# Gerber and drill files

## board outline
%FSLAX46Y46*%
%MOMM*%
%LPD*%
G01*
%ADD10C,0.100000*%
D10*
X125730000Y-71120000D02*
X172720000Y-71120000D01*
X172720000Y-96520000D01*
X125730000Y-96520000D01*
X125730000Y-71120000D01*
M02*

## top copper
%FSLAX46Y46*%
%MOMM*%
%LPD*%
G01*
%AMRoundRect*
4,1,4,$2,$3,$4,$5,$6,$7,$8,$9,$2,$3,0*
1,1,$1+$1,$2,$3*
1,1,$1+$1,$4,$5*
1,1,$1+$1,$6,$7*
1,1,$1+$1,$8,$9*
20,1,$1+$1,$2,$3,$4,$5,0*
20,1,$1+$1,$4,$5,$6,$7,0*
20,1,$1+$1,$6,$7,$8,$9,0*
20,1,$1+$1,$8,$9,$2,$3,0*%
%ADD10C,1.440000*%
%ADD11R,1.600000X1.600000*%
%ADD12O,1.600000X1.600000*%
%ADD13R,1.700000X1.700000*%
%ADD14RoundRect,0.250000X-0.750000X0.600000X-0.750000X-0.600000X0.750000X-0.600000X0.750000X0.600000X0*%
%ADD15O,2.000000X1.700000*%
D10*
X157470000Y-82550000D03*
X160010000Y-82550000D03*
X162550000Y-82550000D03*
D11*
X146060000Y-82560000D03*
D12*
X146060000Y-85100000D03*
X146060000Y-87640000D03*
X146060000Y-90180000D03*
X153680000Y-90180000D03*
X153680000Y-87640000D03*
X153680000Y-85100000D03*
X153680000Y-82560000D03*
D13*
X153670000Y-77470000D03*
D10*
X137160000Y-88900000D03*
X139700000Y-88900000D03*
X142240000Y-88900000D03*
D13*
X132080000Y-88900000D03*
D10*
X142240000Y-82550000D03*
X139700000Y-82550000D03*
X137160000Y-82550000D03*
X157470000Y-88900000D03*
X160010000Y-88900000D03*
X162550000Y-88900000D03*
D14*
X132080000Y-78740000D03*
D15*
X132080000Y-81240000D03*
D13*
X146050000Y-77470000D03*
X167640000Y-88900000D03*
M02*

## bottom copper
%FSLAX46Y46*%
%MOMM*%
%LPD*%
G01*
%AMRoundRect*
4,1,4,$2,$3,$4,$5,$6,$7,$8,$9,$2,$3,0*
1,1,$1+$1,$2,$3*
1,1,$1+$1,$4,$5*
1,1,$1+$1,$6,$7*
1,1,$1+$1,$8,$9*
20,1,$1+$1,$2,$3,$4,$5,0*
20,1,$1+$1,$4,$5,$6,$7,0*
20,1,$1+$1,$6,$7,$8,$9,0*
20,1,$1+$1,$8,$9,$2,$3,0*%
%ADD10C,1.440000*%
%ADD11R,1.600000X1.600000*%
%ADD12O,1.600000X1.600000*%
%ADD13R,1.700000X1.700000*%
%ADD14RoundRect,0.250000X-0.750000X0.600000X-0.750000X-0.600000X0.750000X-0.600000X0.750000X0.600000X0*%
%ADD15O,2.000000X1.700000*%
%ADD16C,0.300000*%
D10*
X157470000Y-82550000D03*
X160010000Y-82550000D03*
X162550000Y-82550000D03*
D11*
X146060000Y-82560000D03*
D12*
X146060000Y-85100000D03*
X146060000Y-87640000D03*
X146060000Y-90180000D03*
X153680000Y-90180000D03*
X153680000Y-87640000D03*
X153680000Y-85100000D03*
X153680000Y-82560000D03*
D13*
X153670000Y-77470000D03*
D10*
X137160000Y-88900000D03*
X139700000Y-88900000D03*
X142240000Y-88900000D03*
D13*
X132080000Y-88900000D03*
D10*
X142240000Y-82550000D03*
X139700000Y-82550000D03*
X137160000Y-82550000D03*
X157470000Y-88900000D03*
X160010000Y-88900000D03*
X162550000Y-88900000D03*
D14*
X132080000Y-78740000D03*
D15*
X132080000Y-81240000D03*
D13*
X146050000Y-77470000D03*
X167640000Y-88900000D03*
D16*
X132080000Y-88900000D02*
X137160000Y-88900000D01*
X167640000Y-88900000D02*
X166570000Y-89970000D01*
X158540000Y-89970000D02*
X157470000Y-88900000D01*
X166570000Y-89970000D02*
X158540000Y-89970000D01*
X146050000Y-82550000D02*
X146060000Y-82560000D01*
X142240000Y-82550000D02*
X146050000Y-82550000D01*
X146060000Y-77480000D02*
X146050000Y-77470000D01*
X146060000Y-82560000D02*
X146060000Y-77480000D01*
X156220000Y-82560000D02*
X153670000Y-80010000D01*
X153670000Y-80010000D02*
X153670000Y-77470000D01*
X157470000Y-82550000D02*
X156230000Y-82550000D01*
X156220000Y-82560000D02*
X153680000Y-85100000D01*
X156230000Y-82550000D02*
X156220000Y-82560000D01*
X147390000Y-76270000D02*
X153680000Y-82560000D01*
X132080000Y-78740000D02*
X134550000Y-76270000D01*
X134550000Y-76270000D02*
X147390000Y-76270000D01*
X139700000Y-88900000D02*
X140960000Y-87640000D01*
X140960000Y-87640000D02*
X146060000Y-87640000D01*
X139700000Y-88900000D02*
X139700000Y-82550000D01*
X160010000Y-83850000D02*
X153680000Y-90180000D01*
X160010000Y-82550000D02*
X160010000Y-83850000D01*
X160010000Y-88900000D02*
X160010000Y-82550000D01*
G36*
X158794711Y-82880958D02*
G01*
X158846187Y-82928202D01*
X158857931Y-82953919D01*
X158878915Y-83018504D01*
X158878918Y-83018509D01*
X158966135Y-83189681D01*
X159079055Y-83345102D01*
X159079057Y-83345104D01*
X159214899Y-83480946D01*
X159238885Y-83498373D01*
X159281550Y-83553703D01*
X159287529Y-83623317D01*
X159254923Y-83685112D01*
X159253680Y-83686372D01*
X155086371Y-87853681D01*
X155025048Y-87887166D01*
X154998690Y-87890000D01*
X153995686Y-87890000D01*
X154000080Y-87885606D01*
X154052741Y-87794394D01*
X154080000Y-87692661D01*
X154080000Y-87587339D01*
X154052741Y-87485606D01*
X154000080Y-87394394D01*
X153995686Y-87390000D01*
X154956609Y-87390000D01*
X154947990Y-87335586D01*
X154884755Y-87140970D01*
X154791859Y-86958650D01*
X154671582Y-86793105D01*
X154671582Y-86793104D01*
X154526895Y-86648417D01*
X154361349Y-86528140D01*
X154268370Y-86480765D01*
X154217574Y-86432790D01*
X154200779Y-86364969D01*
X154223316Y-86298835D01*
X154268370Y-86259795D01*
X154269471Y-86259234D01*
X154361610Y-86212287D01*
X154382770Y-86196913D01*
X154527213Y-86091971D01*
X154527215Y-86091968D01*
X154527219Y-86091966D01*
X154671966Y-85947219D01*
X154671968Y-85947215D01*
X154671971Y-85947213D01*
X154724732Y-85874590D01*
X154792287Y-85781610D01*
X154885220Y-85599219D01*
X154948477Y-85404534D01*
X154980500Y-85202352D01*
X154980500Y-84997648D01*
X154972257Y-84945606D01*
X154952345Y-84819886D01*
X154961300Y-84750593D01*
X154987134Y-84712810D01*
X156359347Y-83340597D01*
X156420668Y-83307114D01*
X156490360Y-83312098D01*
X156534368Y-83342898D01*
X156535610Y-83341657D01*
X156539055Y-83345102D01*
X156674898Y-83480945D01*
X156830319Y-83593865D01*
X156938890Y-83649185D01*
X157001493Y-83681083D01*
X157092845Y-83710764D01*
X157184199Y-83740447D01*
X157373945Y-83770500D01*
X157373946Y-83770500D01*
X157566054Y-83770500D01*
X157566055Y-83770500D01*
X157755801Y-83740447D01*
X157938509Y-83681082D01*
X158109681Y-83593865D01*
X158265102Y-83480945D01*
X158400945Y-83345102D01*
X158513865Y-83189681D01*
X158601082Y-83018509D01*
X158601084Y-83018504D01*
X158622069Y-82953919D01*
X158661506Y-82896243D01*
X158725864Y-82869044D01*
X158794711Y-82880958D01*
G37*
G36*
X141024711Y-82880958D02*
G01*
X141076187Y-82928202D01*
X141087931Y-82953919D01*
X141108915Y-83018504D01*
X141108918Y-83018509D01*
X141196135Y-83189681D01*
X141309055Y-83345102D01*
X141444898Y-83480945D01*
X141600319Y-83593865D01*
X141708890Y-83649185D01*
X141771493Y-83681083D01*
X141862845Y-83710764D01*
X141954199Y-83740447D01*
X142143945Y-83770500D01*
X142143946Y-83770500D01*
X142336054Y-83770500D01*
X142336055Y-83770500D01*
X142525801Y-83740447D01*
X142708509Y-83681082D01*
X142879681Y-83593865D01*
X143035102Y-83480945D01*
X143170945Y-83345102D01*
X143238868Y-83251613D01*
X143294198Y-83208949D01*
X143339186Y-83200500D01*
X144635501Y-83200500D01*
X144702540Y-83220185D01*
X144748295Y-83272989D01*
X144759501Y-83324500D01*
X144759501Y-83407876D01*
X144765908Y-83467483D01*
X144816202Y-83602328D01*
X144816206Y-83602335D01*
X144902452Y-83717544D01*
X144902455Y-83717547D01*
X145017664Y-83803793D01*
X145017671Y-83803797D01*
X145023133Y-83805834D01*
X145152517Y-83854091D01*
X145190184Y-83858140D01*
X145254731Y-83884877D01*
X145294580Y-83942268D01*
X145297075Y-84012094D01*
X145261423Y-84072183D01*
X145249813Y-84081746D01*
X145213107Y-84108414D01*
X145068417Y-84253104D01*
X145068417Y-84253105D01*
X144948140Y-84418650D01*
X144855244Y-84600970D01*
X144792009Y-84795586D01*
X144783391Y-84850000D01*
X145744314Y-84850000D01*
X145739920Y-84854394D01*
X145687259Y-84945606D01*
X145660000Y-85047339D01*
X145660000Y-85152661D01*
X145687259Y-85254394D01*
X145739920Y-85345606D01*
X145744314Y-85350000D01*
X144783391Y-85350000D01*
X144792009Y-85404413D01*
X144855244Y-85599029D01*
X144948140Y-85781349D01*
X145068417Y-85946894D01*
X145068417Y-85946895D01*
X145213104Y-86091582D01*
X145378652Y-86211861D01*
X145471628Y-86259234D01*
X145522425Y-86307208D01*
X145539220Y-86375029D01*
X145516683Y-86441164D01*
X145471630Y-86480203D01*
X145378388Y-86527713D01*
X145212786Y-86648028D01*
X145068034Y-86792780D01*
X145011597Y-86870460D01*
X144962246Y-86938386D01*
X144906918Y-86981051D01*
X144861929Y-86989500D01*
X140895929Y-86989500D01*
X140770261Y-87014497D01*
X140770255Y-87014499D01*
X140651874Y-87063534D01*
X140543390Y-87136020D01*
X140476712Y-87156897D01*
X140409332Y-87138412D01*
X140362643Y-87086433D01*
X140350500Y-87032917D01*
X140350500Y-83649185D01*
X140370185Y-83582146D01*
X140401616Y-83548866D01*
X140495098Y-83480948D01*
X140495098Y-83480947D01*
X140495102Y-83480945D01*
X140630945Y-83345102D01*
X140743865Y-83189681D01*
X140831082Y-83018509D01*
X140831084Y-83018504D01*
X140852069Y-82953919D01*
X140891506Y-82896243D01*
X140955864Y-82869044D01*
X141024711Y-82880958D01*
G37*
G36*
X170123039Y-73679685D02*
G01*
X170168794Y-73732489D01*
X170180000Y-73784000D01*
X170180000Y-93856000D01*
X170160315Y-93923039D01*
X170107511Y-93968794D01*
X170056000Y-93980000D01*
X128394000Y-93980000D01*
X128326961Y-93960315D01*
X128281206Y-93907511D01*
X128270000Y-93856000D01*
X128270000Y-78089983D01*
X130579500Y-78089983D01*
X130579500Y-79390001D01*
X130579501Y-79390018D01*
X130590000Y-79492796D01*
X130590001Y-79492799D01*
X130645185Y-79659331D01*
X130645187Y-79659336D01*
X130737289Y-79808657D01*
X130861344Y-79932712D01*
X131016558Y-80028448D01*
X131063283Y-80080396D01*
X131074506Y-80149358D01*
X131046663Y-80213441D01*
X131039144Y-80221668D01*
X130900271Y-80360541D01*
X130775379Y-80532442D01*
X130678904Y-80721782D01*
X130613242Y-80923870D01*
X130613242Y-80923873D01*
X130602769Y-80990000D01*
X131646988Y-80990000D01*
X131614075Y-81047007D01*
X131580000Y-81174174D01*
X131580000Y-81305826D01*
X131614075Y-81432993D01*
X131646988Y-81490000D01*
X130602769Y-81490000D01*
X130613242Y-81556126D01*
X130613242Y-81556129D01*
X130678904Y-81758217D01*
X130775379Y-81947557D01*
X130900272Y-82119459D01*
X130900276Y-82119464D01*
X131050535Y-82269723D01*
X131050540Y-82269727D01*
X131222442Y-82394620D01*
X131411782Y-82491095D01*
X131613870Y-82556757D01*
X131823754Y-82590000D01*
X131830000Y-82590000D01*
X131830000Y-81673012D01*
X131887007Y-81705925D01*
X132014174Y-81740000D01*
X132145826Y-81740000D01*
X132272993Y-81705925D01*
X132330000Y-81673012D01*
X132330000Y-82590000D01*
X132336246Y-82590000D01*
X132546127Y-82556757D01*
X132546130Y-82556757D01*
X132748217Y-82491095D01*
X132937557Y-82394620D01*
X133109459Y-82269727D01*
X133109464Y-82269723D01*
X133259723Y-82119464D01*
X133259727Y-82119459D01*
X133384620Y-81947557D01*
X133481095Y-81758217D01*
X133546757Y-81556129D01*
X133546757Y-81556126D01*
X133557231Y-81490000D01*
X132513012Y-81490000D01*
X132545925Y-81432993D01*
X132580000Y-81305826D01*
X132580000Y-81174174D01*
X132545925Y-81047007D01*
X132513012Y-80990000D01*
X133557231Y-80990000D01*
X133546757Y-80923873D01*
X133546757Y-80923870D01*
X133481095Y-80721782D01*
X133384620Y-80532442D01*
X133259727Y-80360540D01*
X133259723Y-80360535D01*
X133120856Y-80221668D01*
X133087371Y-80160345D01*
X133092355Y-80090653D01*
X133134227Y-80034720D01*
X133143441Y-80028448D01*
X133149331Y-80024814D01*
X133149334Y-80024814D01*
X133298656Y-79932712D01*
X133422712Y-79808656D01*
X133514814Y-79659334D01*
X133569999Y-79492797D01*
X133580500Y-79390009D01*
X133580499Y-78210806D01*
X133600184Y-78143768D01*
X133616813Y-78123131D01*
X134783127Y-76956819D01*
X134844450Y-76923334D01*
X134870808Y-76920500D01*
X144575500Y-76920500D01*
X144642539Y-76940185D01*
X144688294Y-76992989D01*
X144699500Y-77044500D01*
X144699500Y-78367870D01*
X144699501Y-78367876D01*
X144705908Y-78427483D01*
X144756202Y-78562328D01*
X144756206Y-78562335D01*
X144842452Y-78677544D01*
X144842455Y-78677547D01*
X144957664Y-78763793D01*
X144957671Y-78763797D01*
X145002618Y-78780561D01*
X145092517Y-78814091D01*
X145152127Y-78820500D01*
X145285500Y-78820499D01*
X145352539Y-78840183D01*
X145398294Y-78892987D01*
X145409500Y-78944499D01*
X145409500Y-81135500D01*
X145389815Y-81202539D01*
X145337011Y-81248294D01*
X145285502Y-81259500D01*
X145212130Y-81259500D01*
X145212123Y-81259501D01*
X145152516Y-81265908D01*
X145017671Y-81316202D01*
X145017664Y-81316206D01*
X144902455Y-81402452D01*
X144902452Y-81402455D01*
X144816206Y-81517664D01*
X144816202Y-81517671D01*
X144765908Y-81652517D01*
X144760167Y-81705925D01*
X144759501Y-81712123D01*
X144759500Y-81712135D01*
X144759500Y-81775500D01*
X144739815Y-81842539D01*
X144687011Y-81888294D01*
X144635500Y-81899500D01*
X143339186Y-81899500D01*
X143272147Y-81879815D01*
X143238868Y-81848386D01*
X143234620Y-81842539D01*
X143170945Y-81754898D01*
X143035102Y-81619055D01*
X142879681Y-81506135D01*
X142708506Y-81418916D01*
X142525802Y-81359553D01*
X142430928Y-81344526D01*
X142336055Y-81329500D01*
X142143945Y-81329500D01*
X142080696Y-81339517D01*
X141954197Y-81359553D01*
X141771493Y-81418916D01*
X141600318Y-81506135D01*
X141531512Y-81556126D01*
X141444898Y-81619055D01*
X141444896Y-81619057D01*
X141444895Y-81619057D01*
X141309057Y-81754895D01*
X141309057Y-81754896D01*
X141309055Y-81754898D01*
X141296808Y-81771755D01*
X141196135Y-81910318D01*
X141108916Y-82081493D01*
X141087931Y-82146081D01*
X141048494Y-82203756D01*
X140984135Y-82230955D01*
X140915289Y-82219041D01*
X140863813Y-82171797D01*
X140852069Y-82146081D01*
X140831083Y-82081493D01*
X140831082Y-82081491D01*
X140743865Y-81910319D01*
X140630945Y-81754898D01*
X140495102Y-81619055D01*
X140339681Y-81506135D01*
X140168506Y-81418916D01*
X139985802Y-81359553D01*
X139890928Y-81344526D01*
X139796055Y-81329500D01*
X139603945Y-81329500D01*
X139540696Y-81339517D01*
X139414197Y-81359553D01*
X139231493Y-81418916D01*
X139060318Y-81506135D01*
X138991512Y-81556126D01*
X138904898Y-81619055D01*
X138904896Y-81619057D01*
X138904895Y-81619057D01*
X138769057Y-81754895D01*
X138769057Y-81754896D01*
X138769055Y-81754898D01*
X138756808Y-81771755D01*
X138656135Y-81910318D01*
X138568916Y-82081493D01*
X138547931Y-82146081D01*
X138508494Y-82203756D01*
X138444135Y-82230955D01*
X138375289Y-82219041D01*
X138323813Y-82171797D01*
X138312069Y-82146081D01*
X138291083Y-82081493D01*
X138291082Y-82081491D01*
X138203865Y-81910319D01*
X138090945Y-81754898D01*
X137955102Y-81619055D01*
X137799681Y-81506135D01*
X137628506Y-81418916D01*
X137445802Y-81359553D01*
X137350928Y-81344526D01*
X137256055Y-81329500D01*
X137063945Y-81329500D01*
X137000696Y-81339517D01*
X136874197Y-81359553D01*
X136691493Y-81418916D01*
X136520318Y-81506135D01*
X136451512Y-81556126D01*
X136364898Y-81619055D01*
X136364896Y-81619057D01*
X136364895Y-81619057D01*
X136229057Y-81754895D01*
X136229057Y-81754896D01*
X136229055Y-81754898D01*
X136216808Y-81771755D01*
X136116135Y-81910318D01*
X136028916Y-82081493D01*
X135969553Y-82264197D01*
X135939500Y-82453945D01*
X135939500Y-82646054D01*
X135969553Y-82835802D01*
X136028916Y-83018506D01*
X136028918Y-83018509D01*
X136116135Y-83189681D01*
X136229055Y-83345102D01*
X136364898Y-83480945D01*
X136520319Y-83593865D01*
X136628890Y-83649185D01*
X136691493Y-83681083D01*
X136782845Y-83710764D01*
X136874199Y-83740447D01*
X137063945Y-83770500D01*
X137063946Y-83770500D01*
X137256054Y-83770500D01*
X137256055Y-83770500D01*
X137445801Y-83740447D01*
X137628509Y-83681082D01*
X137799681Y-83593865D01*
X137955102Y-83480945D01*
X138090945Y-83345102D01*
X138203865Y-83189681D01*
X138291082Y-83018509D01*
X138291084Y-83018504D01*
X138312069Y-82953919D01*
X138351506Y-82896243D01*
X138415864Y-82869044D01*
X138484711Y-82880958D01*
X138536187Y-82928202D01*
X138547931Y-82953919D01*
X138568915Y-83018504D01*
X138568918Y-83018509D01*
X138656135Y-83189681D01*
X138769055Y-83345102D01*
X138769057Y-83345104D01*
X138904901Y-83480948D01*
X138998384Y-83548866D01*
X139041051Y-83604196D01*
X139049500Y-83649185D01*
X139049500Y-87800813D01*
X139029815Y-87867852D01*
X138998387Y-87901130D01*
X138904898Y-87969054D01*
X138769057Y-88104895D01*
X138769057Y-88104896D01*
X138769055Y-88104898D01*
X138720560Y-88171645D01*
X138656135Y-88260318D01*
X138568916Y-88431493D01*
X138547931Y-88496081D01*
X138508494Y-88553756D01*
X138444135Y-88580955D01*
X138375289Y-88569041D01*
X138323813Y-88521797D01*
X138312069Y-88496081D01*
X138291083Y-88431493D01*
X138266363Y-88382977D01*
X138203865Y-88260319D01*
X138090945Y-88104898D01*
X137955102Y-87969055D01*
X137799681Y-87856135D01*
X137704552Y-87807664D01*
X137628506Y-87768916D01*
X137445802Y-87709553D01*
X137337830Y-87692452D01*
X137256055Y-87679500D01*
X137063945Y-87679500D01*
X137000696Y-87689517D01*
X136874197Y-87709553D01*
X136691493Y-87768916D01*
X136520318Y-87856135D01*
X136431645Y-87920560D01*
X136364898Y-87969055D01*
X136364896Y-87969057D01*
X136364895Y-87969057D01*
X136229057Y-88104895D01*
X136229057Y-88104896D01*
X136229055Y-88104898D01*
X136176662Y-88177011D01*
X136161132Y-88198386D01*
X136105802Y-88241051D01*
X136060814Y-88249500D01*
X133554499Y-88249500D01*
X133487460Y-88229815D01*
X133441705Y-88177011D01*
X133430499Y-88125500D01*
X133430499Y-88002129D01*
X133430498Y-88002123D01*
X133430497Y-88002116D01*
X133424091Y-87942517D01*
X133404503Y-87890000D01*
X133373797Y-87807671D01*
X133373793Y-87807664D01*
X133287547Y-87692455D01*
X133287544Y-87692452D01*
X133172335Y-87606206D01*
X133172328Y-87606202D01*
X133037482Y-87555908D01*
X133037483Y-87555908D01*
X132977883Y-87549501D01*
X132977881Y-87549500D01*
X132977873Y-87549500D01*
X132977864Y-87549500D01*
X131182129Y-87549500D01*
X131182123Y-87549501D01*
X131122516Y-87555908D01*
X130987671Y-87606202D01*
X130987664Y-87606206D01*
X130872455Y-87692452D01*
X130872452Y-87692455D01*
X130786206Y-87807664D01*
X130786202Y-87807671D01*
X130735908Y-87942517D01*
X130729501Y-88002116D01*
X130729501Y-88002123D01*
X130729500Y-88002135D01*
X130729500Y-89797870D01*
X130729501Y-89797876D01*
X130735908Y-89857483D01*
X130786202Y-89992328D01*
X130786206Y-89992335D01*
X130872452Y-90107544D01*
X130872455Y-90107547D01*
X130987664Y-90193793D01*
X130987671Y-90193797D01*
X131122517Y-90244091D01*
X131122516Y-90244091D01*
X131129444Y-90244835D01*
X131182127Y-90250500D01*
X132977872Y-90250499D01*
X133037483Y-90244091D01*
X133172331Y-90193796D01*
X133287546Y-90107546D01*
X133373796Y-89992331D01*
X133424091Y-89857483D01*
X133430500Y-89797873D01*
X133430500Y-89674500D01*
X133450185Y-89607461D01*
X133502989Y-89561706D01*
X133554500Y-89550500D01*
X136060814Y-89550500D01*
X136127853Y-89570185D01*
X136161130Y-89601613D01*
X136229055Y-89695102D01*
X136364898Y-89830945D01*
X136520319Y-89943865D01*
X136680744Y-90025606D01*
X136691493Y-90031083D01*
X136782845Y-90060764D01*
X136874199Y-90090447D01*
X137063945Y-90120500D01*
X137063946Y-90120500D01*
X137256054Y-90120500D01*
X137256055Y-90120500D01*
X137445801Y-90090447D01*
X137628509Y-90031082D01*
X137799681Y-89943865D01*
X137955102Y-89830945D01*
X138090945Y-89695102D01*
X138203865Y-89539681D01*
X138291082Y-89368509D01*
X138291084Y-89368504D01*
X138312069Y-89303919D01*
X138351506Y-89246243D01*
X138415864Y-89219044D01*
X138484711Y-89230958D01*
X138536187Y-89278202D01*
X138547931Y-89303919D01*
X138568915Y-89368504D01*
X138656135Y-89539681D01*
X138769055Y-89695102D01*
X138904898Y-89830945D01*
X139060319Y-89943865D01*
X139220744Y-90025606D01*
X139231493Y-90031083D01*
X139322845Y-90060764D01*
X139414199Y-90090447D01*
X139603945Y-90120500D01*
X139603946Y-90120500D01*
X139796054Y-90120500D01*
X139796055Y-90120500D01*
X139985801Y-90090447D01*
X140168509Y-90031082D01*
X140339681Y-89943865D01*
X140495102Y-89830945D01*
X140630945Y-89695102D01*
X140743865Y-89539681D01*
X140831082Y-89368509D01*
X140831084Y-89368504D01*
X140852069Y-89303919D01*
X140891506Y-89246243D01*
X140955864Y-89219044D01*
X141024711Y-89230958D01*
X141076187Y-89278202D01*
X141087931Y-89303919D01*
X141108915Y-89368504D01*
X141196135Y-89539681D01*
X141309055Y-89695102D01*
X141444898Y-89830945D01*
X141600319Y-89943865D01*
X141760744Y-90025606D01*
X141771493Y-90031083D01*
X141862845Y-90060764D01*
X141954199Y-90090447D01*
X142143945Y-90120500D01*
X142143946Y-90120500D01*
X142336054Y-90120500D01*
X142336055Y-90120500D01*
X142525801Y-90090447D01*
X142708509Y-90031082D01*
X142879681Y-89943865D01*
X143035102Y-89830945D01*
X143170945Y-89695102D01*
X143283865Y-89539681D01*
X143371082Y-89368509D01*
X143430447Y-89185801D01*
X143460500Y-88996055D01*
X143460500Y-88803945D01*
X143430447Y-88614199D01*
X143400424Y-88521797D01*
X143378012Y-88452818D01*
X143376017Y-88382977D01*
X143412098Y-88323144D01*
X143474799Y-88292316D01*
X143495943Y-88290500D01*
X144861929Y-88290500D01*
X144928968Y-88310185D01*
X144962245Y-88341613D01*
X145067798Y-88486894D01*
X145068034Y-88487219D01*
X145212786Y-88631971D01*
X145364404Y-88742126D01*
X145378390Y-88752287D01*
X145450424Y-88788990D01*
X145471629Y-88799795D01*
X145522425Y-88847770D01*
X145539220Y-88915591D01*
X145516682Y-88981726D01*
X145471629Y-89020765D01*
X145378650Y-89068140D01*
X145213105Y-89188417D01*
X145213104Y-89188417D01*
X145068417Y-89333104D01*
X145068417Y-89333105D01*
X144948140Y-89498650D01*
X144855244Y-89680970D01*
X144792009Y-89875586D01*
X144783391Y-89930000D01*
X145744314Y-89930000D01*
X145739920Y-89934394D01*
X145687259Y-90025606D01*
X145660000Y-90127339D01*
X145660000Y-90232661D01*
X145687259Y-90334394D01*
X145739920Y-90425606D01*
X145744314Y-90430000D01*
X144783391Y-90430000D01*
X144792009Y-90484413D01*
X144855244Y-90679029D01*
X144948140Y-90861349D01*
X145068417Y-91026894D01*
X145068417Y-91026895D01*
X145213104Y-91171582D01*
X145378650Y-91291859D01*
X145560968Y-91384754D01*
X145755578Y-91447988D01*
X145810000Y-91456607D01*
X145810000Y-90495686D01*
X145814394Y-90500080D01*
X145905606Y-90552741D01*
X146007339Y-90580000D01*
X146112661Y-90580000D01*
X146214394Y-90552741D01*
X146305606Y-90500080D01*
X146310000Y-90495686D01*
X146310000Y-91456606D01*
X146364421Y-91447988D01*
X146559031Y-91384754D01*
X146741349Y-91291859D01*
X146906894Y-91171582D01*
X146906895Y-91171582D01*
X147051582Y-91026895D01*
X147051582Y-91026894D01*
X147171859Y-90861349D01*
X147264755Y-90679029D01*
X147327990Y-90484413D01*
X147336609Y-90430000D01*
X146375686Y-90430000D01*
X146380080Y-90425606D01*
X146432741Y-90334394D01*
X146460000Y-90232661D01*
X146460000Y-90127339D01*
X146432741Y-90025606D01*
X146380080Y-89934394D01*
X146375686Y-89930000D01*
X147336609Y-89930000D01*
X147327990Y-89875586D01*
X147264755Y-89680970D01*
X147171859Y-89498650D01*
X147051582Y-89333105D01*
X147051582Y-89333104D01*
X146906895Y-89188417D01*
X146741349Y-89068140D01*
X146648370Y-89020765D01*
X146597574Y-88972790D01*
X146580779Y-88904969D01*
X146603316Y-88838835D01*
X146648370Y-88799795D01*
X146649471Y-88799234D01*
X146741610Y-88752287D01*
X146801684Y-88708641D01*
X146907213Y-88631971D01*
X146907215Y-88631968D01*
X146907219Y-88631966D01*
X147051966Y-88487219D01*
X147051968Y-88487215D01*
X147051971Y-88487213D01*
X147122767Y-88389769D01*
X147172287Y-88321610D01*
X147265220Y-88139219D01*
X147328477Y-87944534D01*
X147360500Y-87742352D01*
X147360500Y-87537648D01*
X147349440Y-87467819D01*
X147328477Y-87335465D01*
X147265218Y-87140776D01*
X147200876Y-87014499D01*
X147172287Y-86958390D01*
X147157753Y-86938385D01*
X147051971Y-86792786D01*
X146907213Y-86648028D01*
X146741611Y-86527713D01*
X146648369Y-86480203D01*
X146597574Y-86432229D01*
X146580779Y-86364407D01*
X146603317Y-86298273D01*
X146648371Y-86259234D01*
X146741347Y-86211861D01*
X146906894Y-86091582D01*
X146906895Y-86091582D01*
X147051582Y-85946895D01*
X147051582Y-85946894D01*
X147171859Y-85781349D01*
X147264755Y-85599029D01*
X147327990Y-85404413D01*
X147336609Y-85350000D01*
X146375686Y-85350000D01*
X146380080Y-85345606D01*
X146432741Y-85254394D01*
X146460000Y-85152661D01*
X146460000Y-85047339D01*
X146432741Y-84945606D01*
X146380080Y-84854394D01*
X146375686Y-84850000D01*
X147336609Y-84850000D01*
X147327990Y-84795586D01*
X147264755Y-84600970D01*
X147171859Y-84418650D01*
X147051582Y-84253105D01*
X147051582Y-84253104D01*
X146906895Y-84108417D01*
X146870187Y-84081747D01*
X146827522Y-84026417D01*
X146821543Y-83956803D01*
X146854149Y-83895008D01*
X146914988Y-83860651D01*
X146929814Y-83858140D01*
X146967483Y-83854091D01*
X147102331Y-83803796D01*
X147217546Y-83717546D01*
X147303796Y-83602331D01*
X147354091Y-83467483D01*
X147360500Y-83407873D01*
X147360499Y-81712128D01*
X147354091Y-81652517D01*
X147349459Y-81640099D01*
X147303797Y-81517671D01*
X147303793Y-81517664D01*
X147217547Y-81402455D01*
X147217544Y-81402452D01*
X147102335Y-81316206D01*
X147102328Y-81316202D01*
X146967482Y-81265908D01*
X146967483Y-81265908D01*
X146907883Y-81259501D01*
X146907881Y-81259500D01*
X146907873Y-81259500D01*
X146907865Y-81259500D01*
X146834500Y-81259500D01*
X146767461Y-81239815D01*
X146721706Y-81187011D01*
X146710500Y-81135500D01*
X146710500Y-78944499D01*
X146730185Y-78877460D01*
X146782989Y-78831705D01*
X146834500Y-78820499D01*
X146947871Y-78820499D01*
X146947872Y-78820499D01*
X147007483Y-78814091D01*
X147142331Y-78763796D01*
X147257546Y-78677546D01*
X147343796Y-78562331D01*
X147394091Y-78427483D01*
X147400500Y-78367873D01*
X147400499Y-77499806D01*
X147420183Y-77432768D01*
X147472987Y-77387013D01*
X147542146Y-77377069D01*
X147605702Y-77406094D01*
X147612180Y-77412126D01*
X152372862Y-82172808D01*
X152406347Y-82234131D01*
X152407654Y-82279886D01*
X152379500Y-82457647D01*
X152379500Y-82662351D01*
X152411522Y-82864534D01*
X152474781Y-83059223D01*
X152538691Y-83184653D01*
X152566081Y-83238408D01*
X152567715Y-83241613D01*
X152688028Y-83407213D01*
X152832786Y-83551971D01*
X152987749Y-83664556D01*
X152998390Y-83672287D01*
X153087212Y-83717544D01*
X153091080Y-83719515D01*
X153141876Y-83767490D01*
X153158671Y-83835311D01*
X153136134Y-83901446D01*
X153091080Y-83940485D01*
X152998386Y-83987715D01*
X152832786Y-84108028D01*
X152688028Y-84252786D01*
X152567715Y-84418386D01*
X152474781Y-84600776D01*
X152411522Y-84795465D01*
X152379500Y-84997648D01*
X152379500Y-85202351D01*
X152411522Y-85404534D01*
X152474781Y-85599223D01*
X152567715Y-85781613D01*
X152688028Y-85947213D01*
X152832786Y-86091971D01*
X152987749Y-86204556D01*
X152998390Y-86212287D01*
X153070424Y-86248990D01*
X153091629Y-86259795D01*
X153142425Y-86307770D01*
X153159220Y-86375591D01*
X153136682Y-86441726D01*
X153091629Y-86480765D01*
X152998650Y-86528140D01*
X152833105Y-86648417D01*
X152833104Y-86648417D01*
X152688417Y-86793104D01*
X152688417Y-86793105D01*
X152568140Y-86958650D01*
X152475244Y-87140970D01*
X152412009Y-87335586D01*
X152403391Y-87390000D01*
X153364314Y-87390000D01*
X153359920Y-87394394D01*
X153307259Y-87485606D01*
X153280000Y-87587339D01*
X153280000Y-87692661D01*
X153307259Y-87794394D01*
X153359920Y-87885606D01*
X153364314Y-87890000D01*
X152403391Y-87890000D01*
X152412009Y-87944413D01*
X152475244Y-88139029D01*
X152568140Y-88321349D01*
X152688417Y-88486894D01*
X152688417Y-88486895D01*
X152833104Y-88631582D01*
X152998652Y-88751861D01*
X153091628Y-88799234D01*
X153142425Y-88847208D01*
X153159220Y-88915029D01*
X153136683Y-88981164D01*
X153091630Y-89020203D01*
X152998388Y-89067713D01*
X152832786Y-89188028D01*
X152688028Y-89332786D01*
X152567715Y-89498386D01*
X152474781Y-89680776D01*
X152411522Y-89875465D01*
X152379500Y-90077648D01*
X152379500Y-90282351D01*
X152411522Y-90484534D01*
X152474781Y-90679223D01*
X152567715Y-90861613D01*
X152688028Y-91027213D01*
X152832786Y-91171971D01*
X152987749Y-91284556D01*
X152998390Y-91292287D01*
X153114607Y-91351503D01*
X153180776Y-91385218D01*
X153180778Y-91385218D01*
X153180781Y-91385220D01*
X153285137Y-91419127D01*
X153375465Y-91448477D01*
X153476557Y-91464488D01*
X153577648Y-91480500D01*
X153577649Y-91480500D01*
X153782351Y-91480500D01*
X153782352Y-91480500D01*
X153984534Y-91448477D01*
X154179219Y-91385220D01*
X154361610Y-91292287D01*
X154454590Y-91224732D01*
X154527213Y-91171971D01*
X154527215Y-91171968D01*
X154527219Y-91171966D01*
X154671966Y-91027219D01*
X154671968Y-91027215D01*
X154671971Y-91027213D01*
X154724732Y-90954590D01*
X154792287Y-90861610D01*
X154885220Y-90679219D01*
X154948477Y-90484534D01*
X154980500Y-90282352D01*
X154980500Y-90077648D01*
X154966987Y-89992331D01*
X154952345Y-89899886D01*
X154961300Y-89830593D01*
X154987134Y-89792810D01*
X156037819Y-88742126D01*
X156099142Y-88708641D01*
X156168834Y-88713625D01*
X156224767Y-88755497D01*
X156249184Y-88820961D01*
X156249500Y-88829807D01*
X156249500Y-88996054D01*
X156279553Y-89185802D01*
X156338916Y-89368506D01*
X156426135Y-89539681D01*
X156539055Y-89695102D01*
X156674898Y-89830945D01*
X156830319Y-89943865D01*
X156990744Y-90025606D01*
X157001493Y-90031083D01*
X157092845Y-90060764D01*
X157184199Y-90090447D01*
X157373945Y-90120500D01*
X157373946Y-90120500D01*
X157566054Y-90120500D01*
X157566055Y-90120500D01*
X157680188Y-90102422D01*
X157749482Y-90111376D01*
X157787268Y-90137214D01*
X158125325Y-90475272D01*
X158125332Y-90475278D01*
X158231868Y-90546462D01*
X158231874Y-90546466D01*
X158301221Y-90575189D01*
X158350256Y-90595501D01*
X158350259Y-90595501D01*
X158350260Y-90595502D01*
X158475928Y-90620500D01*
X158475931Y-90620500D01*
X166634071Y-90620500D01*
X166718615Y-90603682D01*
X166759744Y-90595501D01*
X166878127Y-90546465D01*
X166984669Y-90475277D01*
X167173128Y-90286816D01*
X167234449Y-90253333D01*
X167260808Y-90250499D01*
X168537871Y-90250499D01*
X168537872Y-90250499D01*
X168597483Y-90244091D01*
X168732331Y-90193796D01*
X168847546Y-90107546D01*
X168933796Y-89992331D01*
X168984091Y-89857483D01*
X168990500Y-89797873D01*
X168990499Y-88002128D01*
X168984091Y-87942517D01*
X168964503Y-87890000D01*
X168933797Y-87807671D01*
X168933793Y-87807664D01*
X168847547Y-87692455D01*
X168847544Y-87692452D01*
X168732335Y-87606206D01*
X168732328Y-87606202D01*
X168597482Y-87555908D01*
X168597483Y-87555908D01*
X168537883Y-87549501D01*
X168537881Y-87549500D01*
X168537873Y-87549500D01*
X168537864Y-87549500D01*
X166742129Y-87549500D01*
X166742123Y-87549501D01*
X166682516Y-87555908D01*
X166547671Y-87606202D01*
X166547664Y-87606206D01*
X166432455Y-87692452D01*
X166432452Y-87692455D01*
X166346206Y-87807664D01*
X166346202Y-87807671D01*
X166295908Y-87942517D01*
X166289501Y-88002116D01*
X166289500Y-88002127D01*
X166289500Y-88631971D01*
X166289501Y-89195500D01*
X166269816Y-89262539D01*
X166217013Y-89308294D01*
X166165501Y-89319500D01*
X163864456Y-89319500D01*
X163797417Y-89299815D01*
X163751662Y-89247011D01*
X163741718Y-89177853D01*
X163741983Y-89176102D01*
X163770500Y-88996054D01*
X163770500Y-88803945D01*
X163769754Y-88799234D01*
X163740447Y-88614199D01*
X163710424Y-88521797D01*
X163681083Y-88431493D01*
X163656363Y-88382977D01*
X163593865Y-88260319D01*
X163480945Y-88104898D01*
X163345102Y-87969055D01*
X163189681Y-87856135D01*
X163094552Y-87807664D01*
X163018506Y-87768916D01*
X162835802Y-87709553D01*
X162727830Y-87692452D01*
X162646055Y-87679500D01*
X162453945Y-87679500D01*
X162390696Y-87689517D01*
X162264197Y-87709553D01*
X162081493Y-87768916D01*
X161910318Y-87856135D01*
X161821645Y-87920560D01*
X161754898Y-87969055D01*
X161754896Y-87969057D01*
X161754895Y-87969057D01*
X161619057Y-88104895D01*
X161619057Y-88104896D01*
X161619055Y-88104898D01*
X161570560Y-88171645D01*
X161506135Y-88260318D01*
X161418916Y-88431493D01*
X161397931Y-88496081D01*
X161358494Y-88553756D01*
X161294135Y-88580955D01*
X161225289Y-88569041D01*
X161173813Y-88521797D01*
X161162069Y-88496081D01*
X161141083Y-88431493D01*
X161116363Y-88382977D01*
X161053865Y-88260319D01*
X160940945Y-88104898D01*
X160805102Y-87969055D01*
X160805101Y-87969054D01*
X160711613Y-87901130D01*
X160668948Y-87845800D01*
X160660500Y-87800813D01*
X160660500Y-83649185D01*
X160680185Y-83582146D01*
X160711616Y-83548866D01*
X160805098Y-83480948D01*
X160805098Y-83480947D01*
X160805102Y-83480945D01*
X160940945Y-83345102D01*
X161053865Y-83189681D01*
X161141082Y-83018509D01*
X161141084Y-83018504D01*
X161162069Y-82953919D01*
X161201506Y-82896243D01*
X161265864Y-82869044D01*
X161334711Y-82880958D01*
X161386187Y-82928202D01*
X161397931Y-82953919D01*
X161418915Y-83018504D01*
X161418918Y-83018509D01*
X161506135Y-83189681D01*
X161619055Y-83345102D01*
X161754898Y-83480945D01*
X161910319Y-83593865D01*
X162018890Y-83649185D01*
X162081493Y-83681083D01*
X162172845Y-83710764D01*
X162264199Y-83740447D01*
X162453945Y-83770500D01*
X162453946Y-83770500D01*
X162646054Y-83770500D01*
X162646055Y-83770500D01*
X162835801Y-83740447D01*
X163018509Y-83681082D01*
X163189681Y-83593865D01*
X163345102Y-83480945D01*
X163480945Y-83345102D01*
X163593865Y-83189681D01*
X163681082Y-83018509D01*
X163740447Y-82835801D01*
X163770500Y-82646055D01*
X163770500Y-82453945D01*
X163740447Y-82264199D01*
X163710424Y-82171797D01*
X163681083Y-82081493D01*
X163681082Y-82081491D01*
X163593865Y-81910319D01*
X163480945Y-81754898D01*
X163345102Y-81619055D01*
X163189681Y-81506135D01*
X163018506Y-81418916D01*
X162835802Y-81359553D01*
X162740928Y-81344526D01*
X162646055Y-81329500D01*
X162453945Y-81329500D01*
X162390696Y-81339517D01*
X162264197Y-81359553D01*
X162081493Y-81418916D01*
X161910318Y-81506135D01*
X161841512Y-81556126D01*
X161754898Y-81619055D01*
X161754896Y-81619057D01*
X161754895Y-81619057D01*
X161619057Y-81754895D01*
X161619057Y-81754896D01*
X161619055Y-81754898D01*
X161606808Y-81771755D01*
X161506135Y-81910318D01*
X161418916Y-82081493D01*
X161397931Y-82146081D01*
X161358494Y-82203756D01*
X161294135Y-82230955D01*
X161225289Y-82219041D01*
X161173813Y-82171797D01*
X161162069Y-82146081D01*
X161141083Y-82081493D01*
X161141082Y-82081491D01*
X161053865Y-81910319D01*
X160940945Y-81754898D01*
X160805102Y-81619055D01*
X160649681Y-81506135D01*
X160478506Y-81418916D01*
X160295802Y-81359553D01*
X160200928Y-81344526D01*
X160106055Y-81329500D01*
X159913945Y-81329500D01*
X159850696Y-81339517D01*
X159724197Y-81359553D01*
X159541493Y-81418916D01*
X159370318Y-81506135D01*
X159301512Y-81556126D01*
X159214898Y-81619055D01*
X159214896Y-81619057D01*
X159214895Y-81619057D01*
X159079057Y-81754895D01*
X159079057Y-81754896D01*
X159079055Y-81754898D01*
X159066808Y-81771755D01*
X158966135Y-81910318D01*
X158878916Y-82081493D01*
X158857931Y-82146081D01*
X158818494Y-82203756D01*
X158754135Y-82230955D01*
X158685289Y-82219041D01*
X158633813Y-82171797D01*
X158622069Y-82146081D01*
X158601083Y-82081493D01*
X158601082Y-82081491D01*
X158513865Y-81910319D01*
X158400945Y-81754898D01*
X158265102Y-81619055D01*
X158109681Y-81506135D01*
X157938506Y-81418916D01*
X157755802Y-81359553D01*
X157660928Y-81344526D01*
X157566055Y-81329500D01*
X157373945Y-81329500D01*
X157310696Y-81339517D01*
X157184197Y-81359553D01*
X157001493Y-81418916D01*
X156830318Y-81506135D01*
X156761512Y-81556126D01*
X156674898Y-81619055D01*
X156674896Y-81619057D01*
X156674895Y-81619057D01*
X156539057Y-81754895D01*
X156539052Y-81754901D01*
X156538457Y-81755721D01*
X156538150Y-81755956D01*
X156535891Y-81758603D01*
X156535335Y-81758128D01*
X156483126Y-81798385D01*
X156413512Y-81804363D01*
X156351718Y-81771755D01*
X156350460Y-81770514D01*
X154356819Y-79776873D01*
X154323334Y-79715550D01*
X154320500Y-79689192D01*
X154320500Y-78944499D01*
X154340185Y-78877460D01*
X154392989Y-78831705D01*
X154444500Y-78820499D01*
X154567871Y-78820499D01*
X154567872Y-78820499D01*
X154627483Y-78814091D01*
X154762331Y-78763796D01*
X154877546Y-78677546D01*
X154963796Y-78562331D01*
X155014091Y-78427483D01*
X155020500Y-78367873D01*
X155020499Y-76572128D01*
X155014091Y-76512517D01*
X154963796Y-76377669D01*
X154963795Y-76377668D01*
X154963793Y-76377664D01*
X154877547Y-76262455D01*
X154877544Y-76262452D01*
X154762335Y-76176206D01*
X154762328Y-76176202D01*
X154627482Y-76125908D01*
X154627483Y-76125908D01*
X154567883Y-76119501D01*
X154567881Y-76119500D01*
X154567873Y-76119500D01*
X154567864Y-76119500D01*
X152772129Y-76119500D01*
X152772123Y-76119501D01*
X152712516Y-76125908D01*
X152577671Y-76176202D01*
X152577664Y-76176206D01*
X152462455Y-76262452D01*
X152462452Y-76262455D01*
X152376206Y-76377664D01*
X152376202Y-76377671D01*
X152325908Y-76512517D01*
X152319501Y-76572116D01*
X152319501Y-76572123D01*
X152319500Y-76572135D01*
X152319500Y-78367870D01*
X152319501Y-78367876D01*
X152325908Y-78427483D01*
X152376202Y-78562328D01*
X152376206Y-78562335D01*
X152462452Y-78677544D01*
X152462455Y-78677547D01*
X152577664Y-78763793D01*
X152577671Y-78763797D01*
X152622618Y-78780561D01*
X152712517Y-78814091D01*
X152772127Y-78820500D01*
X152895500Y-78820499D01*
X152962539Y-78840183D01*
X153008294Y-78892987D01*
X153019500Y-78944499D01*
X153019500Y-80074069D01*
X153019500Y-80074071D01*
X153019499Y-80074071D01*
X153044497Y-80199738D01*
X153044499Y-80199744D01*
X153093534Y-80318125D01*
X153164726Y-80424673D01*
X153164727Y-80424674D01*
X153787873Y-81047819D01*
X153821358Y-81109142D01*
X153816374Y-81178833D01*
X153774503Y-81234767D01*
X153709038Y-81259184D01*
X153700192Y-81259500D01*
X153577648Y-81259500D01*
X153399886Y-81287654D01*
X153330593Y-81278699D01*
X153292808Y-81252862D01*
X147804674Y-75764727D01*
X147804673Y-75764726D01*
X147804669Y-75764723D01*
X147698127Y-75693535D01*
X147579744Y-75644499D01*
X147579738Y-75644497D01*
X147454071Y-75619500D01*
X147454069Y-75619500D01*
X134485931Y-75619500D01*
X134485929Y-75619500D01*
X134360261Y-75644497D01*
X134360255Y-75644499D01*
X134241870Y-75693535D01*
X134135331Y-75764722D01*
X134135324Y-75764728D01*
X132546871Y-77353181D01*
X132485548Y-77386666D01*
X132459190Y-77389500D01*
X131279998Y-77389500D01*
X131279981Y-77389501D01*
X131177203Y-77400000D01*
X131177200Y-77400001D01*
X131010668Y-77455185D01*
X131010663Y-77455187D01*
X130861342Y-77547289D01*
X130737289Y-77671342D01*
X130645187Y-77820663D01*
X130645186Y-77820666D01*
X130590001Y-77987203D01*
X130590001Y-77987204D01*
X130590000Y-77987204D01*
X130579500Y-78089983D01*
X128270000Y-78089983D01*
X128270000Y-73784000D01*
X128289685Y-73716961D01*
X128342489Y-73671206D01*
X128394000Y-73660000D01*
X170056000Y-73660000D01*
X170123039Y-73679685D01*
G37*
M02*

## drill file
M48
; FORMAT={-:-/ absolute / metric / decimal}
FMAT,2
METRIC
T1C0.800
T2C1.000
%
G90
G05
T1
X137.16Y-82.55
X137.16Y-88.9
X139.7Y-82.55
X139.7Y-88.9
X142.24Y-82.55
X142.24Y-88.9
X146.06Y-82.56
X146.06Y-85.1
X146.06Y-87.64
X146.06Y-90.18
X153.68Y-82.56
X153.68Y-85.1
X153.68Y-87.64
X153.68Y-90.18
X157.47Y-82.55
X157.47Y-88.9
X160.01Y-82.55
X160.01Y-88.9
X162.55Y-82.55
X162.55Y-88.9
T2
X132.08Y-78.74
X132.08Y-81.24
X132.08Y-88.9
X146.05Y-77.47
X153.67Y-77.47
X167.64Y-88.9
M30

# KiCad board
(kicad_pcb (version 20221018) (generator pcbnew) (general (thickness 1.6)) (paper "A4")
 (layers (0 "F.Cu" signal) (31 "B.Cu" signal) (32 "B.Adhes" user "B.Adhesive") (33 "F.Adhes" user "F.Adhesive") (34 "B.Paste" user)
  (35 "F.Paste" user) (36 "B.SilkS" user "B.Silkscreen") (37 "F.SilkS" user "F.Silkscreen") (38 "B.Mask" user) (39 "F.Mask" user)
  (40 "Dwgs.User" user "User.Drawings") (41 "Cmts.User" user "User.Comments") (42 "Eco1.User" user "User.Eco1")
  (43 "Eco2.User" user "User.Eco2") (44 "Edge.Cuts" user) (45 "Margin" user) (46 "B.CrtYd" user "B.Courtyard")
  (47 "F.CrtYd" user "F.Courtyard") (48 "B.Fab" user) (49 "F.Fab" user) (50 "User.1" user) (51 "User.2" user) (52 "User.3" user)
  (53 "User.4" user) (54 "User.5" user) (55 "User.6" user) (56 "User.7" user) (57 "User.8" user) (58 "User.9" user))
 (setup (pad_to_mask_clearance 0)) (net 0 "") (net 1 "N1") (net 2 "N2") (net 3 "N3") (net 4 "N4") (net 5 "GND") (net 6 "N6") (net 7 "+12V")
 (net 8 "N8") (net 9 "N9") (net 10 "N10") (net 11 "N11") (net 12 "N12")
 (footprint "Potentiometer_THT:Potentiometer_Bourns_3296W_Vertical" (layer "F.Cu") (at 157.47 82.55 180)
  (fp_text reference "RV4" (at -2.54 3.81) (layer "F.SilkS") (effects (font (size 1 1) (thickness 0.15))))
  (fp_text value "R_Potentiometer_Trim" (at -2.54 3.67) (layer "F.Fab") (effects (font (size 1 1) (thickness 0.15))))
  (pad "1" thru_hole circle (at 0 0 180) (size 1.44 1.44) (drill 0.8) (layers "*.Cu" "*.Mask") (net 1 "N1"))
  (pad "2" thru_hole circle (at -2.54 0 180) (size 1.44 1.44) (drill 0.8) (layers "*.Cu" "*.Mask") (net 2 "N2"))
  (pad "3" thru_hole circle (at -5.08 0 180) (size 1.44 1.44) (drill 0.8) (layers "*.Cu" "*.Mask") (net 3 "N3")))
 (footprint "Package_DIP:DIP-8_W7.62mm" (layer "F.Cu") (at 146.06 82.56)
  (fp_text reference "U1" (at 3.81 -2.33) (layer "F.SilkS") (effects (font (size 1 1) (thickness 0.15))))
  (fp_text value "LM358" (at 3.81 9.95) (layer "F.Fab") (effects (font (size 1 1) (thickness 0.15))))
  (pad "1" thru_hole rect (at 0 0) (size 1.6 1.6) (drill 0.8) (layers "*.Cu" "*.Mask") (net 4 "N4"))
  (pad "2" thru_hole oval (at 0 2.54) (size 1.6 1.6) (drill 0.8) (layers "*.Cu" "*.Mask") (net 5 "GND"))
  (pad "3" thru_hole oval (at 0 5.08) (size 1.6 1.6) (drill 0.8) (layers "*.Cu" "*.Mask") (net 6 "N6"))
  (pad "4" thru_hole oval (at 0 7.62) (size 1.6 1.6) (drill 0.8) (layers "*.Cu" "*.Mask") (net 5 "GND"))
  (pad "5" thru_hole oval (at 7.62 7.62) (size 1.6 1.6) (drill 0.8) (layers "*.Cu" "*.Mask") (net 2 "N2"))
  (pad "6" thru_hole oval (at 7.62 5.08) (size 1.6 1.6) (drill 0.8) (layers "*.Cu" "*.Mask") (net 5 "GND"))
  (pad "7" thru_hole oval (at 7.62 2.54) (size 1.6 1.6) (drill 0.8) (layers "*.Cu" "*.Mask") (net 1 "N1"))
  (pad "8" thru_hole oval (at 7.62 0) (size 1.6 1.6) (drill 0.8) (layers "*.Cu" "*.Mask") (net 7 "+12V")))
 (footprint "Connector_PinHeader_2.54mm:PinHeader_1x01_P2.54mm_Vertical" (layer "F.Cu") (at 153.67 77.47)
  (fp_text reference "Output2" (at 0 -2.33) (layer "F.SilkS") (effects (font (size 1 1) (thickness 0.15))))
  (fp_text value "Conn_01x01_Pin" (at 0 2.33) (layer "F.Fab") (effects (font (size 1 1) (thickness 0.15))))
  (pad "1" thru_hole rect (at 0 0) (size 1.7 1.7) (drill 1) (layers "*.Cu" "*.Mask") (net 1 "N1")))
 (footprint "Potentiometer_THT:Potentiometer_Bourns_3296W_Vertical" (layer "F.Cu") (at 137.16 88.9 180)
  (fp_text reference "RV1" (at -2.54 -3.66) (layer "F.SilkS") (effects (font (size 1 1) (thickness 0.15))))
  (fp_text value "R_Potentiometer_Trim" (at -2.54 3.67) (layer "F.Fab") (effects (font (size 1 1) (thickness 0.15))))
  (pad "1" thru_hole circle (at 0 0 180) (size 1.44 1.44) (drill 0.8) (layers "*.Cu" "*.Mask") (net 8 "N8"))
  (pad "2" thru_hole circle (at -2.54 0 180) (size 1.44 1.44) (drill 0.8) (layers "*.Cu" "*.Mask") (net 6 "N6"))
  (pad "3" thru_hole circle (at -5.08 0 180) (size 1.44 1.44) (drill 0.8) (layers "*.Cu" "*.Mask") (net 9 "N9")))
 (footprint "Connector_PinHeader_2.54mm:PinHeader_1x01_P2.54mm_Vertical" (layer "F.Cu") (at 132.08 88.9)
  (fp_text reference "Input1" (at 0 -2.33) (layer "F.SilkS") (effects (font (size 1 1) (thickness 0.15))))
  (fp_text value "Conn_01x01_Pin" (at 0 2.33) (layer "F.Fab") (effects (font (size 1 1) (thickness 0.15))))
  (pad "1" thru_hole rect (at 0 0) (size 1.7 1.7) (drill 1) (layers "*.Cu" "*.Mask") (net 8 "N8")))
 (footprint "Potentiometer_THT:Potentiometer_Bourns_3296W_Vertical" (layer "F.Cu") (at 142.24 82.55)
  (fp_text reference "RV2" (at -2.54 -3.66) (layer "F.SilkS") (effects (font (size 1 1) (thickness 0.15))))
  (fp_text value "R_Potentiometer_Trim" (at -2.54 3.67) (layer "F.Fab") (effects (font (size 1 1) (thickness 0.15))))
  (pad "1" thru_hole circle (at 0 0) (size 1.44 1.44) (drill 0.8) (layers "*.Cu" "*.Mask") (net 4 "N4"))
  (pad "2" thru_hole circle (at -2.54 0) (size 1.44 1.44) (drill 0.8) (layers "*.Cu" "*.Mask") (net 6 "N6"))
  (pad "3" thru_hole circle (at -5.08 0) (size 1.44 1.44) (drill 0.8) (layers "*.Cu" "*.Mask") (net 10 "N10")))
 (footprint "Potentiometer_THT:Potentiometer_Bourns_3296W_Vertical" (layer "F.Cu") (at 157.47 88.9 180)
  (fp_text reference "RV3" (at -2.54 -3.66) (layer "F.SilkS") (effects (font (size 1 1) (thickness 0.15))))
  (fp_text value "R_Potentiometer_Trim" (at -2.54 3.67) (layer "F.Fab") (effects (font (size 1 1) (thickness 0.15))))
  (pad "1" thru_hole circle (at 0 0 180) (size 1.44 1.44) (drill 0.8) (layers "*.Cu" "*.Mask") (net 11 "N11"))
  (pad "2" thru_hole circle (at -2.54 0 180) (size 1.44 1.44) (drill 0.8) (layers "*.Cu" "*.Mask") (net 2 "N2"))
  (pad "3" thru_hole circle (at -5.08 0 180) (size 1.44 1.44) (drill 0.8) (layers "*.Cu" "*.Mask") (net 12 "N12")))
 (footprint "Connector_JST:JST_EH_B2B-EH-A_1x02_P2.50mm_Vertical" (layer "F.Cu") (at 132.08 78.74 -90)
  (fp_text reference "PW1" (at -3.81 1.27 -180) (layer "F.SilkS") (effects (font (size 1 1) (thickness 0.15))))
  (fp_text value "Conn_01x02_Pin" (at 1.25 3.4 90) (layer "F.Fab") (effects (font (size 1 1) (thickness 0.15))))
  (pad "1" thru_hole roundrect (at 0 0 270) (size 1.7 2) (drill 1) (layers "*.Cu" "*.Mask") (roundrect_rratio 0.147059) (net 7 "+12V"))
  (pad "2" thru_hole oval (at 2.5 0 270) (size 1.7 2) (drill 1) (layers "*.Cu" "*.Mask") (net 5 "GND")))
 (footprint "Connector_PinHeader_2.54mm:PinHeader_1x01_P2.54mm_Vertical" (layer "F.Cu") (at 146.05 77.47)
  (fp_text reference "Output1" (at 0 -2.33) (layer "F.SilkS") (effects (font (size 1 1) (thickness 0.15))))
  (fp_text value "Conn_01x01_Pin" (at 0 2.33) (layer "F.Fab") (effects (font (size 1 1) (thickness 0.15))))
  (pad "1" thru_hole rect (at 0 0) (size 1.7 1.7) (drill 1) (layers "*.Cu" "*.Mask") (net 4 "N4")))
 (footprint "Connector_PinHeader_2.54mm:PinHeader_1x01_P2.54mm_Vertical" (layer "F.Cu") (at 167.64 88.9)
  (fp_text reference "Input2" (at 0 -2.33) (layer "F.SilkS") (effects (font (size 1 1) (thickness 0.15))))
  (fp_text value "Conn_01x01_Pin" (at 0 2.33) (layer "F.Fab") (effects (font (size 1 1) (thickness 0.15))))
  (pad "1" thru_hole rect (at 0 0) (size 1.7 1.7) (drill 1) (layers "*.Cu" "*.Mask") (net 11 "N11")))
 (gr_rect (start 125.73 71.12) (end 172.72 96.52) (stroke (width 0.1) (type default)) (fill none) (layer "Edge.Cuts"))
 (segment (start 132.08 88.9) (end 137.16 88.9) (width 0.3) (layer "B.Cu") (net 8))
 (segment (start 167.64 88.9) (end 166.57 89.97) (width 0.3) (layer "B.Cu") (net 11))
 (segment (start 158.54 89.97) (end 157.47 88.9) (width 0.3) (layer "B.Cu") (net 11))
 (segment (start 166.57 89.97) (end 158.54 89.97) (width 0.3) (layer "B.Cu") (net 11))
 (segment (start 146.05 82.55) (end 146.06 82.56) (width 0.3) (layer "B.Cu") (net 4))
 (segment (start 142.24 82.55) (end 146.05 82.55) (width 0.3) (layer "B.Cu") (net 4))
 (segment (start 146.06 77.48) (end 146.05 77.47) (width 0.3) (layer "B.Cu") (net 4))
 (segment (start 146.06 82.56) (end 146.06 77.48) (width 0.3) (layer "B.Cu") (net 4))
 (segment (start 156.22 82.56) (end 153.67 80.01) (width 0.3) (layer "B.Cu") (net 1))
 (segment (start 153.67 80.01) (end 153.67 77.47) (width 0.3) (layer "B.Cu") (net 1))
 (segment (start 157.47 82.55) (end 156.23 82.55) (width 0.3) (layer "B.Cu") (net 1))
 (segment (start 156.22 82.56) (end 153.68 85.1) (width 0.3) (layer "B.Cu") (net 1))
 (segment (start 156.23 82.55) (end 156.22 82.56) (width 0.3) (layer "B.Cu") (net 1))
 (segment (start 147.39 76.27) (end 153.68 82.56) (width 0.3) (layer "B.Cu") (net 7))
 (segment (start 132.08 78.74) (end 134.55 76.27) (width 0.3) (layer "B.Cu") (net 7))
 (segment (start 134.55 76.27) (end 147.39 76.27) (width 0.3) (layer "B.Cu") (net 7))
 (segment (start 139.7 88.9) (end 140.96 87.64) (width 0.3) (layer "B.Cu") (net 6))
 (segment (start 140.96 87.64) (end 146.06 87.64) (width 0.3) (layer "B.Cu") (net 6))
 (segment (start 139.7 88.9) (end 139.7 82.55) (width 0.3) (layer "B.Cu") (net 6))
 (segment (start 160.01 83.85) (end 153.68 90.18) (width 0.3) (layer "B.Cu") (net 2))
 (segment (start 160.01 82.55) (end 160.01 83.85) (width 0.3) (layer "B.Cu") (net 2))
 (segment (start 160.01 88.9) (end 160.01 82.55) (width 0.3) (layer "B.Cu") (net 2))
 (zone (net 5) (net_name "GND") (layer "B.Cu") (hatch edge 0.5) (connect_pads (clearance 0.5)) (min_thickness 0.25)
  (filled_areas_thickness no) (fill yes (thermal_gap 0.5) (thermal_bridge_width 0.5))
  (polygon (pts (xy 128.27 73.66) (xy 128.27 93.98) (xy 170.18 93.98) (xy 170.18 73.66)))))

